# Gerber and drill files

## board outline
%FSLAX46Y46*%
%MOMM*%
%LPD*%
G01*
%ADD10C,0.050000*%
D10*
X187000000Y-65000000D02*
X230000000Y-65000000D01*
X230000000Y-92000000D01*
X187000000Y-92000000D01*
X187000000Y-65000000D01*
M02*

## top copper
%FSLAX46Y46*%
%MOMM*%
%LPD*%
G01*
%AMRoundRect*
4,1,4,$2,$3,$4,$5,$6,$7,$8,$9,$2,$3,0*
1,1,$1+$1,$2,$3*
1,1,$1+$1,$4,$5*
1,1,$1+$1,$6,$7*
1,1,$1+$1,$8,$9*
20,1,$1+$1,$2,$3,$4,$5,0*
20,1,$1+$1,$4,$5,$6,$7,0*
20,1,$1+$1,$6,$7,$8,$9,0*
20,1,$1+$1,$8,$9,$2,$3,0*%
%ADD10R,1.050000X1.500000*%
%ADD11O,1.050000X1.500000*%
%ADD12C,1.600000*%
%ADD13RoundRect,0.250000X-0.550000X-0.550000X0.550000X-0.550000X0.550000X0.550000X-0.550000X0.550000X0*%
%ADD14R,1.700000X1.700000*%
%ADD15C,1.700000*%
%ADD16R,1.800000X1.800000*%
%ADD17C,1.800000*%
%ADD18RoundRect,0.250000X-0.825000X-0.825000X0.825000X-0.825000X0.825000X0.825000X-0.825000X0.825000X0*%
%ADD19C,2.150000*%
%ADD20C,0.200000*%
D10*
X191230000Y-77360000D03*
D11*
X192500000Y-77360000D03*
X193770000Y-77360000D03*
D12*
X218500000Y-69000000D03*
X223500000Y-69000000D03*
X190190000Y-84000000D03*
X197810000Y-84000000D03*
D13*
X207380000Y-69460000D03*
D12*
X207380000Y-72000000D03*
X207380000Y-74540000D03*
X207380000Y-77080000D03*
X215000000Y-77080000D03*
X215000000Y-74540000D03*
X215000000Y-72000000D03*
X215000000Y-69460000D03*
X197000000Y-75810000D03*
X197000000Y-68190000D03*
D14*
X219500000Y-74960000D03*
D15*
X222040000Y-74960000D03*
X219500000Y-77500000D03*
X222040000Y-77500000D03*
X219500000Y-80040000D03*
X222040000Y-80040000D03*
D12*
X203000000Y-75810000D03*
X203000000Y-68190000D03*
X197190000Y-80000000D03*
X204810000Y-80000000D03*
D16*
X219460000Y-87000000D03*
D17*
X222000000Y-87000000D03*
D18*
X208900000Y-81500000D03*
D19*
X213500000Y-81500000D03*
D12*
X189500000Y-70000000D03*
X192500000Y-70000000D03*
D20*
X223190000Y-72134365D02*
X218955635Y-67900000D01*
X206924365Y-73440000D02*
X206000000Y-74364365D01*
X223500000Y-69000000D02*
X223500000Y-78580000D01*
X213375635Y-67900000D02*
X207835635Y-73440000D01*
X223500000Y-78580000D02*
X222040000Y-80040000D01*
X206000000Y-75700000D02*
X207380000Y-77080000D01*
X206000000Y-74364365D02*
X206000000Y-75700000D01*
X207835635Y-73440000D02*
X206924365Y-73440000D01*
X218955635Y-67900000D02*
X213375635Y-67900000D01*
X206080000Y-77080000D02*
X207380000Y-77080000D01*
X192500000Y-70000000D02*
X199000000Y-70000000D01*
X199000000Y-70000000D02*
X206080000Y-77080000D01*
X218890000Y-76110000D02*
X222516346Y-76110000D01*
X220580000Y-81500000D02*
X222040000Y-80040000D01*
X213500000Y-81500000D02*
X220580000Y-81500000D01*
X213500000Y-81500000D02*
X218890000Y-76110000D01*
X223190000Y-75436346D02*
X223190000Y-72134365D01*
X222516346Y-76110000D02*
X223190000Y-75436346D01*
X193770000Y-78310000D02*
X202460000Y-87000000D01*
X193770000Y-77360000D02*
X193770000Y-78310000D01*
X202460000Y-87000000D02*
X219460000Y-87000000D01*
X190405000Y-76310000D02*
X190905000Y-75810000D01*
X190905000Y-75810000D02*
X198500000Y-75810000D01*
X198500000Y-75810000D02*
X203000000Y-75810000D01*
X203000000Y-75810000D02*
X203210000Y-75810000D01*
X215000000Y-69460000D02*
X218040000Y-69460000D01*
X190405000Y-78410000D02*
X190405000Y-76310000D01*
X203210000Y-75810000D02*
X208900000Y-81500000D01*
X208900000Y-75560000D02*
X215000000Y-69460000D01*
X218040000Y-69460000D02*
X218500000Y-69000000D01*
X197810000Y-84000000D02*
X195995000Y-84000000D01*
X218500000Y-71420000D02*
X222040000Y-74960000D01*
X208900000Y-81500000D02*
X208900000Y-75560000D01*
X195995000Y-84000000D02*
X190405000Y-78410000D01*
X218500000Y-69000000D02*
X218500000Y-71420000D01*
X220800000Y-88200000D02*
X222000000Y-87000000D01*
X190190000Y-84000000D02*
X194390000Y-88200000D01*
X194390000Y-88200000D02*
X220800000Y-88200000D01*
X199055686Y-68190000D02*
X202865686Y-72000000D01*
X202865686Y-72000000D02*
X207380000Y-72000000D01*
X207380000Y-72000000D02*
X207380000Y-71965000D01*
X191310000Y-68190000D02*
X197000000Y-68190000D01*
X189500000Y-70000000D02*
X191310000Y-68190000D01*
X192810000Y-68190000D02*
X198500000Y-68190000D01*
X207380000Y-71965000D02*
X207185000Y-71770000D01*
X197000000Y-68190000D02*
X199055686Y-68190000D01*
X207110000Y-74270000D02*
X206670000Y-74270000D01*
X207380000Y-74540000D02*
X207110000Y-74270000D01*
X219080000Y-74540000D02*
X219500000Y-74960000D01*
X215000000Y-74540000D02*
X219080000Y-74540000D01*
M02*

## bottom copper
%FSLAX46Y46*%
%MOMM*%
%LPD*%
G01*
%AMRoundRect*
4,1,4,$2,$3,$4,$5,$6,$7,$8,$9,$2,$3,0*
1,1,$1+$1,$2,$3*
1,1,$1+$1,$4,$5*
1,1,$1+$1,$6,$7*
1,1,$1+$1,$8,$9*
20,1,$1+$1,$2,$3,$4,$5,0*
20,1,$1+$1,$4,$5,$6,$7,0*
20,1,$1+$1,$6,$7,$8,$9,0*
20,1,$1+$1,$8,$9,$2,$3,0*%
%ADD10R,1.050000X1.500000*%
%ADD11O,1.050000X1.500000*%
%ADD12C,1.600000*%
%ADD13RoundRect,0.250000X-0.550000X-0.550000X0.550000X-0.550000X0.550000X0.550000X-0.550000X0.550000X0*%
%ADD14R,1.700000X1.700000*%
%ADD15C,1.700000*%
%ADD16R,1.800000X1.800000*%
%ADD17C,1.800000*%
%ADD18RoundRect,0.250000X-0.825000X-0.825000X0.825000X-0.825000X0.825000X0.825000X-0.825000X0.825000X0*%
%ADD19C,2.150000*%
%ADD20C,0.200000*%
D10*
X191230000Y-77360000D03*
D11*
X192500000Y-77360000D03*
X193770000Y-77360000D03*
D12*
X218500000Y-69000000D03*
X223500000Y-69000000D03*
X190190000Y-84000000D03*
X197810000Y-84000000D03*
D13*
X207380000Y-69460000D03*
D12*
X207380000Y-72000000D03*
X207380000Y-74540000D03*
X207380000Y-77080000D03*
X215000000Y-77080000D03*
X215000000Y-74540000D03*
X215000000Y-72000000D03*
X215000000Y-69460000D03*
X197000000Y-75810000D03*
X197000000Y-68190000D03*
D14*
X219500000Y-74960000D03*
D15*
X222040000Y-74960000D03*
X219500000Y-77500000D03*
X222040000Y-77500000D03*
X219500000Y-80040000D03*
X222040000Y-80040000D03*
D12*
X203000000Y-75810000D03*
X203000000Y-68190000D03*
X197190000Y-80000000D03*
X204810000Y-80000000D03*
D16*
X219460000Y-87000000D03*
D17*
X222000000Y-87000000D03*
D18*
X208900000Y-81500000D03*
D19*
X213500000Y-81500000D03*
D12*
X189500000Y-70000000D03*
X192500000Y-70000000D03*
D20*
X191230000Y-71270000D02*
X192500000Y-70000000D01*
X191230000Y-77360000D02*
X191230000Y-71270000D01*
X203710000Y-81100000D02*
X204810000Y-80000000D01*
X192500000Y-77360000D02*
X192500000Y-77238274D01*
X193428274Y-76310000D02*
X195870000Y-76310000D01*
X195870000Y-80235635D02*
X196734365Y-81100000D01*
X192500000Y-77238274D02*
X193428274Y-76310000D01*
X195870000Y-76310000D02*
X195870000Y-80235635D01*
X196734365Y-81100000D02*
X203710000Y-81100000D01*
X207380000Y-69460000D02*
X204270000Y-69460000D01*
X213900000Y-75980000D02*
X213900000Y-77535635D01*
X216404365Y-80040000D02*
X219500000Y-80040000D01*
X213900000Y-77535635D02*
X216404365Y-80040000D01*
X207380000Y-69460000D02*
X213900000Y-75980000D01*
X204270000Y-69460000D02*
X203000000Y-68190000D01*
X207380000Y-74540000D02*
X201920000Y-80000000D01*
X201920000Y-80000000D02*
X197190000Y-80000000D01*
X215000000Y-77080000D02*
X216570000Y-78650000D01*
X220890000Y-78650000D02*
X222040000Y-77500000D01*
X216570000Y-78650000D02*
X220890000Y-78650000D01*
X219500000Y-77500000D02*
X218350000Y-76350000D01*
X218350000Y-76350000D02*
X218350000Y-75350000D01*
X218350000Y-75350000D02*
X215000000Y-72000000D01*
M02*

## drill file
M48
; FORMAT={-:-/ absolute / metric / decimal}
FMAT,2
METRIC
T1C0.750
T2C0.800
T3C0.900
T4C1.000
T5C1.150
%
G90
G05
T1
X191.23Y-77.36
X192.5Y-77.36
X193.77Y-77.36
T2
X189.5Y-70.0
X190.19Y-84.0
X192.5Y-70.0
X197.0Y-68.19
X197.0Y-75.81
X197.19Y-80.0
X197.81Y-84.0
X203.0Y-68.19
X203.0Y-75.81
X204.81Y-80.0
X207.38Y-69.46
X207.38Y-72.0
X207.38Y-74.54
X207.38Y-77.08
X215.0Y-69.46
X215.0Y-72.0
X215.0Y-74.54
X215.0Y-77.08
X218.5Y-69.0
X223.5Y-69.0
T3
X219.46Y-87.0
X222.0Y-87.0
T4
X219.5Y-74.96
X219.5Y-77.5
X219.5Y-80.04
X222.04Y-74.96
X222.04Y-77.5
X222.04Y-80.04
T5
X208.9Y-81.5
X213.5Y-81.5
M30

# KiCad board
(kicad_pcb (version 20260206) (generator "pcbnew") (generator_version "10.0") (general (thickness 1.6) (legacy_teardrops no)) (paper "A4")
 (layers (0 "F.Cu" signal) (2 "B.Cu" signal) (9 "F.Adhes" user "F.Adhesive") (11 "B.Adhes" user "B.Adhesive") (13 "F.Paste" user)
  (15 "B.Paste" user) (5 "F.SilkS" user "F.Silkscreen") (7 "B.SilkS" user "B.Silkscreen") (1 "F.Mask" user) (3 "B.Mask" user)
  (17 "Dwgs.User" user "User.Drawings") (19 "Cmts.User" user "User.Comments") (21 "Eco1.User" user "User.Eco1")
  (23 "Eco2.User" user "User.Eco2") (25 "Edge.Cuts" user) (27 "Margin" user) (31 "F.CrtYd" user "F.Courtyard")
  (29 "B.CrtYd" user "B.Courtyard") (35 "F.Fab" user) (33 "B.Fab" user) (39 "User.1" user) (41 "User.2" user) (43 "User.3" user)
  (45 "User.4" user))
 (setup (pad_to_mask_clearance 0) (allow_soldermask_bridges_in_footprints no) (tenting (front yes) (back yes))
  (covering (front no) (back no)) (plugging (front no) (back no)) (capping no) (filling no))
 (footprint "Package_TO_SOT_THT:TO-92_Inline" (layer "F.Cu") (at 191.23 77.36)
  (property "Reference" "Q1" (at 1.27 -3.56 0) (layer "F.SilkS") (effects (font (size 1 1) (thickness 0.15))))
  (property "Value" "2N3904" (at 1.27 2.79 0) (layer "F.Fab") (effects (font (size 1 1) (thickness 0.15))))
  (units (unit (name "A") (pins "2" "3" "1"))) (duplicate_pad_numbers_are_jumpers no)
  (pad "1" thru_hole rect (at 0 0) (size 1.05 1.5) (drill 0.75) (layers "*.Cu" "*.Mask") (remove_unused_layers no) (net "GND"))
  (pad "2" thru_hole oval (at 1.27 0) (size 1.05 1.5) (drill 0.75) (layers "*.Cu" "*.Mask") (remove_unused_layers no) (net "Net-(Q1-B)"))
  (pad "3" thru_hole oval (at 2.54 0) (size 1.05 1.5) (drill 0.75) (layers "*.Cu" "*.Mask") (remove_unused_layers no) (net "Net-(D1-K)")))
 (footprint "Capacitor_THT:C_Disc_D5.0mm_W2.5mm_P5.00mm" (layer "F.Cu") (at 218.5 69)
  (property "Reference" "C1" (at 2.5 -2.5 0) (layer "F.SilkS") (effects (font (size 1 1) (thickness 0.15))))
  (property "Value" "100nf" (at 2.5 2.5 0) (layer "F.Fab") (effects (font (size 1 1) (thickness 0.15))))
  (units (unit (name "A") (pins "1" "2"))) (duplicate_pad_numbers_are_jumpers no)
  (pad "1" thru_hole circle (at 0 0) (size 1.6 1.6) (drill 0.8) (layers "*.Cu" "*.Mask") (remove_unused_layers no) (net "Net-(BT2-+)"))
  (pad "2" thru_hole circle (at 5 0) (size 1.6 1.6) (drill 0.8) (layers "*.Cu" "*.Mask") (remove_unused_layers no) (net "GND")))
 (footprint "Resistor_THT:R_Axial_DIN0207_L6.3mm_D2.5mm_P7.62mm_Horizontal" (layer "F.Cu") (at 190.19 84)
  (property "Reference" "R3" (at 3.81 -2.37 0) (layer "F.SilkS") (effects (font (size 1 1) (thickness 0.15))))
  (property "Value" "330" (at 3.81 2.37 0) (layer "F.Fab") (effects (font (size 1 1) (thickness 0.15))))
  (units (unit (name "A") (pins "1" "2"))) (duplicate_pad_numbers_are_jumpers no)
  (pad "1" thru_hole circle (at 0 0) (size 1.6 1.6) (drill 0.8) (layers "*.Cu" "*.Mask") (remove_unused_layers no) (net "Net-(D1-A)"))
  (pad "2" thru_hole circle (at 7.62 0) (size 1.6 1.6) (drill 0.8) (layers "*.Cu" "*.Mask") (remove_unused_layers no) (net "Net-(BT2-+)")))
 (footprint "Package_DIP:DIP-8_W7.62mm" (layer "F.Cu") (at 207.38 69.46)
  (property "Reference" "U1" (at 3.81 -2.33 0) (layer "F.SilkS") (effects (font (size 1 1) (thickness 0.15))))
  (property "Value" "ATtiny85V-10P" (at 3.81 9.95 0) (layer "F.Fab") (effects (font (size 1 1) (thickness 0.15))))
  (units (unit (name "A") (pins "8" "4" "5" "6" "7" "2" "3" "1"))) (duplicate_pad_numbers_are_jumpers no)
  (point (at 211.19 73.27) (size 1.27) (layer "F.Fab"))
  (pad "1" thru_hole roundrect (at 0 0) (size 1.6 1.6) (drill 0.8) (layers "*.Cu" "*.Mask") (remove_unused_layers no)
   (roundrect_rratio 0.15625) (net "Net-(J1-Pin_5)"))
  (pad "2" thru_hole circle (at 0 2.54) (size 1.6 1.6) (drill 0.8) (layers "*.Cu" "*.Mask") (remove_unused_layers no)
   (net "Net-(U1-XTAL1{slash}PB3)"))
  (pad "3" thru_hole circle (at 0 5.08) (size 1.6 1.6) (drill 0.8) (layers "*.Cu" "*.Mask") (remove_unused_layers no)
   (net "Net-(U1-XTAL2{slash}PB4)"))
  (pad "4" thru_hole circle (at 0 7.62) (size 1.6 1.6) (drill 0.8) (layers "*.Cu" "*.Mask") (remove_unused_layers no) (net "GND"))
  (pad "5" thru_hole circle (at 7.62 7.62) (size 1.6 1.6) (drill 0.8) (layers "*.Cu" "*.Mask") (remove_unused_layers no)
   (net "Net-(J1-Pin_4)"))
  (pad "6" thru_hole circle (at 7.62 5.08) (size 1.6 1.6) (drill 0.8) (layers "*.Cu" "*.Mask") (remove_unused_layers no)
   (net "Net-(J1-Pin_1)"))
  (pad "7" thru_hole circle (at 7.62 2.54) (size 1.6 1.6) (drill 0.8) (layers "*.Cu" "*.Mask") (remove_unused_layers no)
   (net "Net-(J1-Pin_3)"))
  (pad "8" thru_hole circle (at 7.62 0) (size 1.6 1.6) (drill 0.8) (layers "*.Cu" "*.Mask") (remove_unused_layers no) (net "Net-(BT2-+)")))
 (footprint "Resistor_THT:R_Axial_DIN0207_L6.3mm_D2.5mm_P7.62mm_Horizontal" (layer "F.Cu") (at 197 75.81 90)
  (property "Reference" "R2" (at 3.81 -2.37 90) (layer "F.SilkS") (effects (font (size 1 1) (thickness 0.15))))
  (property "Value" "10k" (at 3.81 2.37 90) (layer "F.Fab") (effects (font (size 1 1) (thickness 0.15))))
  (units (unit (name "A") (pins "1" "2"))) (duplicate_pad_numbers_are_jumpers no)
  (pad "1" thru_hole circle (at 0 0 90) (size 1.6 1.6) (drill 0.8) (layers "*.Cu" "*.Mask") (remove_unused_layers no) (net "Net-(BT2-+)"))
  (pad "2" thru_hole circle (at 7.62 0 90) (size 1.6 1.6) (drill 0.8) (layers "*.Cu" "*.Mask") (remove_unused_layers no)
   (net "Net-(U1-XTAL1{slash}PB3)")))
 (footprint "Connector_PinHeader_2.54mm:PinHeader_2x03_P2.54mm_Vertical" (layer "F.Cu") (at 219.5 74.96)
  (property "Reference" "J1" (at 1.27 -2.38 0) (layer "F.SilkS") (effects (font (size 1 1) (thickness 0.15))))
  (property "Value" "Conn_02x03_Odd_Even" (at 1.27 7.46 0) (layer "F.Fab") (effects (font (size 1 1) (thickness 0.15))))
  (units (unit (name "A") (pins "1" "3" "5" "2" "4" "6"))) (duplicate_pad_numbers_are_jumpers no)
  (pad "1" thru_hole rect (at 0 0) (size 1.7 1.7) (drill 1) (layers "*.Cu" "*.Mask") (remove_unused_layers no) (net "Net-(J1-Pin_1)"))
  (pad "2" thru_hole circle (at 2.54 0) (size 1.7 1.7) (drill 1) (layers "*.Cu" "*.Mask") (remove_unused_layers no) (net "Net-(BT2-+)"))
  (pad "3" thru_hole circle (at 0 2.54) (size 1.7 1.7) (drill 1) (layers "*.Cu" "*.Mask") (remove_unused_layers no) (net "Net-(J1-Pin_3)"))
  (pad "4" thru_hole circle (at 2.54 2.54) (size 1.7 1.7) (drill 1) (layers "*.Cu" "*.Mask") (remove_unused_layers no)
   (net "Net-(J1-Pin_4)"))
  (pad "5" thru_hole circle (at 0 5.08) (size 1.7 1.7) (drill 1) (layers "*.Cu" "*.Mask") (remove_unused_layers no) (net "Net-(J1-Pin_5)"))
  (pad "6" thru_hole circle (at 2.54 5.08) (size 1.7 1.7) (drill 1) (layers "*.Cu" "*.Mask") (remove_unused_layers no) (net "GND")))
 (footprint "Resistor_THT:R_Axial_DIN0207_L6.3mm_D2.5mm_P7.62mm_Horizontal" (layer "F.Cu") (at 203 75.81 90)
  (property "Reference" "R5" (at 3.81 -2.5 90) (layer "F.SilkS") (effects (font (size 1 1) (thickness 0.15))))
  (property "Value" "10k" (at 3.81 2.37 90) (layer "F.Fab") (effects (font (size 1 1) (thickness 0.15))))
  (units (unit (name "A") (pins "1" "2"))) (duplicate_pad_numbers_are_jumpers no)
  (pad "1" thru_hole circle (at 0 0 90) (size 1.6 1.6) (drill 0.8) (layers "*.Cu" "*.Mask") (remove_unused_layers no) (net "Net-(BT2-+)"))
  (pad "2" thru_hole circle (at 7.62 0 90) (size 1.6 1.6) (drill 0.8) (layers "*.Cu" "*.Mask") (remove_unused_layers no)
   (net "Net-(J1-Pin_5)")))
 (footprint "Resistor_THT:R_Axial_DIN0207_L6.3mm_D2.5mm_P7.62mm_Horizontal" (layer "F.Cu") (at 197.19 80)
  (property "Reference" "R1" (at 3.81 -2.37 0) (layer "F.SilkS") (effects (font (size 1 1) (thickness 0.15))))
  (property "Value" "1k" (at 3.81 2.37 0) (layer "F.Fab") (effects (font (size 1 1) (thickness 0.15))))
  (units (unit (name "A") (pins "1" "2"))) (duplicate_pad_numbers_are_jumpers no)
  (pad "1" thru_hole circle (at 0 0) (size 1.6 1.6) (drill 0.8) (layers "*.Cu" "*.Mask") (remove_unused_layers no)
   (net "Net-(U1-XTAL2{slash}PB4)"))
  (pad "2" thru_hole circle (at 7.62 0) (size 1.6 1.6) (drill 0.8) (layers "*.Cu" "*.Mask") (remove_unused_layers no) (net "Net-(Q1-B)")))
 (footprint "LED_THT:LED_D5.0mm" (layer "F.Cu") (at 219.46 87)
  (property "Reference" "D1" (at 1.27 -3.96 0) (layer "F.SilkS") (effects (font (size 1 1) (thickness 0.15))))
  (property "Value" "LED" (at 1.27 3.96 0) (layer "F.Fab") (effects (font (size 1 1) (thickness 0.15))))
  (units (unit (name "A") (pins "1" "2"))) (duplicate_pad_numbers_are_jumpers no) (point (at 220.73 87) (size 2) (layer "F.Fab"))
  (pad "1" thru_hole rect (at 0 0) (size 1.8 1.8) (drill 0.9) (layers "*.Cu" "*.Mask") (remove_unused_layers no) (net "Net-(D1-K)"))
  (pad "2" thru_hole circle (at 2.54 0) (size 1.8 1.8) (drill 0.9) (layers "*.Cu" "*.Mask") (remove_unused_layers no) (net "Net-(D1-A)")))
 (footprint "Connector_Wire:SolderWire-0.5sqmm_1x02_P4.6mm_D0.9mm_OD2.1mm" (layer "F.Cu") (at 208.9 81.5)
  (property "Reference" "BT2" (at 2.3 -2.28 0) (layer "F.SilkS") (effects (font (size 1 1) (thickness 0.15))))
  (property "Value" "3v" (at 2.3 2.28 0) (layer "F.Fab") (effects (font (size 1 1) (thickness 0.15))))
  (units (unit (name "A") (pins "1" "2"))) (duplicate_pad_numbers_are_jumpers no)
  (pad "1" thru_hole roundrect (at 0 0) (size 2.15 2.15) (drill 1.15) (layers "*.Cu" "*.Mask") (remove_unused_layers no)
   (roundrect_rratio 0.116279) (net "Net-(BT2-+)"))
  (pad "2" thru_hole circle (at 4.6 0) (size 2.15 2.15) (drill 1.15) (layers "*.Cu" "*.Mask") (remove_unused_layers no) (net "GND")))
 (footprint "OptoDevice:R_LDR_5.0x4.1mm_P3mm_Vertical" (layer "F.Cu") (at 189.5 70)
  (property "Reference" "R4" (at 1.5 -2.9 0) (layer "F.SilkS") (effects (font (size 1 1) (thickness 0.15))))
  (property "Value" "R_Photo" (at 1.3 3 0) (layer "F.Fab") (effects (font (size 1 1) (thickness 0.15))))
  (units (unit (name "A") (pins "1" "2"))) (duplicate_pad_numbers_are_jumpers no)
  (pad "1" thru_hole circle (at 0 0) (size 1.6 1.6) (drill 0.8) (layers "*.Cu" "*.Mask") (remove_unused_layers no)
   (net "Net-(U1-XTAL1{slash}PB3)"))
  (pad "2" thru_hole circle (at 3 0) (size 1.6 1.6) (drill 0.8) (layers "*.Cu" "*.Mask") (remove_unused_layers no) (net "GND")))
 (gr_rect (start 187 65) (end 230 92) (stroke (width 0.05) (type default)) (fill no) (layer "Edge.Cuts"))
 (segment (start 223.19 72.134365) (end 218.955635 67.9) (width 0.2) (layer "F.Cu") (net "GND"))
 (segment (start 206.924365 73.44) (end 206 74.364365) (width 0.2) (layer "F.Cu") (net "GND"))
 (segment (start 223.5 69) (end 223.5 78.58) (width 0.2) (layer "F.Cu") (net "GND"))
 (segment (start 213.375635 67.9) (end 207.835635 73.44) (width 0.2) (layer "F.Cu") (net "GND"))
 (segment (start 223.5 78.58) (end 222.04 80.04) (width 0.2) (layer "F.Cu") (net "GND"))
 (segment (start 206 75.7) (end 207.38 77.08) (width 0.2) (layer "F.Cu") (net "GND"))
 (segment (start 206 74.364365) (end 206 75.7) (width 0.2) (layer "F.Cu") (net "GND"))
 (segment (start 207.835635 73.44) (end 206.924365 73.44) (width 0.2) (layer "F.Cu") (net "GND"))
 (segment (start 218.955635 67.9) (end 213.375635 67.9) (width 0.2) (layer "F.Cu") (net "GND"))
 (segment (start 206.08 77.08) (end 207.38 77.08) (width 0.2) (layer "F.Cu") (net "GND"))
 (segment (start 192.5 70) (end 199 70) (width 0.2) (layer "F.Cu") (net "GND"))
 (segment (start 199 70) (end 206.08 77.08) (width 0.2) (layer "F.Cu") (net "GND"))
 (segment (start 218.89 76.11) (end 222.516346 76.11) (width 0.2) (layer "F.Cu") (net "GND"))
 (segment (start 220.58 81.5) (end 222.04 80.04) (width 0.2) (layer "F.Cu") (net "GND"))
 (segment (start 213.5 81.5) (end 220.58 81.5) (width 0.2) (layer "F.Cu") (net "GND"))
 (segment (start 213.5 81.5) (end 218.89 76.11) (width 0.2) (layer "F.Cu") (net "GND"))
 (segment (start 223.19 75.436346) (end 223.19 72.134365) (width 0.2) (layer "F.Cu") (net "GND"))
 (segment (start 222.516346 76.11) (end 223.19 75.436346) (width 0.2) (layer "F.Cu") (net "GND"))
 (segment (start 191.23 71.27) (end 192.5 70) (width 0.2) (layer "B.Cu") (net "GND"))
 (segment (start 191.23 77.36) (end 191.23 71.27) (width 0.2) (layer "B.Cu") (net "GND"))
 (segment (start 203.71 81.1) (end 204.81 80) (width 0.2) (layer "B.Cu") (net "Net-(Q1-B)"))
 (segment (start 192.5 77.36) (end 192.5 77.238274) (width 0.2) (layer "B.Cu") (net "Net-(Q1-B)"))
 (segment (start 193.428274 76.31) (end 195.87 76.31) (width 0.2) (layer "B.Cu") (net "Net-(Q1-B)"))
 (segment (start 195.87 80.235635) (end 196.734365 81.1) (width 0.2) (layer "B.Cu") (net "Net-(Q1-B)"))
 (segment (start 192.5 77.238274) (end 193.428274 76.31) (width 0.2) (layer "B.Cu") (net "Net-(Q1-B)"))
 (segment (start 195.87 76.31) (end 195.87 80.235635) (width 0.2) (layer "B.Cu") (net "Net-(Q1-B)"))
 (segment (start 196.734365 81.1) (end 203.71 81.1) (width 0.2) (layer "B.Cu") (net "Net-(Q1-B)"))
 (segment (start 193.77 78.31) (end 202.46 87) (width 0.2) (layer "F.Cu") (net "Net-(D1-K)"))
 (segment (start 193.77 77.36) (end 193.77 78.31) (width 0.2) (layer "F.Cu") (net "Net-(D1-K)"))
 (segment (start 202.46 87) (end 219.46 87) (width 0.2) (layer "F.Cu") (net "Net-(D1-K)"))
 (segment (start 190.405 76.31) (end 190.905 75.81) (width 0.2) (layer "F.Cu") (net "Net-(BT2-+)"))
 (segment (start 190.905 75.81) (end 198.5 75.81) (width 0.2) (layer "F.Cu") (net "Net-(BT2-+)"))
 (segment (start 198.5 75.81) (end 203 75.81) (width 0.2) (layer "F.Cu") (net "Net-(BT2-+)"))
 (segment (start 203 75.81) (end 203.21 75.81) (width 0.2) (layer "F.Cu") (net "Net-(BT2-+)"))
 (segment (start 215 69.46) (end 218.04 69.46) (width 0.2) (layer "F.Cu") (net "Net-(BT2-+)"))
 (segment (start 190.405 78.41) (end 190.405 76.31) (width 0.2) (layer "F.Cu") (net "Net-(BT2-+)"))
 (segment (start 203.21 75.81) (end 208.9 81.5) (width 0.2) (layer "F.Cu") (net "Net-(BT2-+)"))
 (segment (start 208.9 75.56) (end 215 69.46) (width 0.2) (layer "F.Cu") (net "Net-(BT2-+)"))
 (segment (start 218.04 69.46) (end 218.5 69) (width 0.2) (layer "F.Cu") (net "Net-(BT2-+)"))
 (segment (start 197.81 84) (end 195.995 84) (width 0.2) (layer "F.Cu") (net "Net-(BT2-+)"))
 (segment (start 218.5 71.42) (end 222.04 74.96) (width 0.2) (layer "F.Cu") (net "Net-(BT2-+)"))
 (segment (start 208.9 81.5) (end 208.9 75.56) (width 0.2) (layer "F.Cu") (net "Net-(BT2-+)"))
 (segment (start 195.995 84) (end 190.405 78.41) (width 0.2) (layer "F.Cu") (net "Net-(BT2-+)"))
 (segment (start 218.5 69) (end 218.5 71.42) (width 0.2) (layer "F.Cu") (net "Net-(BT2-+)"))
 (segment (start 220.8 88.2) (end 222 87) (width 0.2) (layer "F.Cu") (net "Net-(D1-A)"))
 (segment (start 190.19 84) (end 194.39 88.2) (width 0.2) (layer "F.Cu") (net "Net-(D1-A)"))
 (segment (start 194.39 88.2) (end 220.8 88.2) (width 0.2) (layer "F.Cu") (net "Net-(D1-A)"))
 (segment (start 207.38 69.46) (end 204.27 69.46) (width 0.2) (layer "B.Cu") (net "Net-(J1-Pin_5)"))
 (segment (start 213.9 75.98) (end 213.9 77.535635) (width 0.2) (layer "B.Cu") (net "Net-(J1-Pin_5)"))
 (segment (start 216.404365 80.04) (end 219.5 80.04) (width 0.2) (layer "B.Cu") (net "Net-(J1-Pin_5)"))
 (segment (start 213.9 77.535635) (end 216.404365 80.04) (width 0.2) (layer "B.Cu") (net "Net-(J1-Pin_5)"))
 (segment (start 207.38 69.46) (end 213.9 75.98) (width 0.2) (layer "B.Cu") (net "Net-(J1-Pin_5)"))
 (segment (start 204.27 69.46) (end 203 68.19) (width 0.2) (layer "B.Cu") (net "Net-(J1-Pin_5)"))
 (segment (start 199.055686 68.19) (end 202.865686 72) (width 0.2) (layer "F.Cu") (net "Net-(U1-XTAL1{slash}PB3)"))
 (segment (start 202.865686 72) (end 207.38 72) (width 0.2) (layer "F.Cu") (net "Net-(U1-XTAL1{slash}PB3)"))
 (segment (start 207.38 72) (end 207.38 71.965) (width 0.2) (layer "F.Cu") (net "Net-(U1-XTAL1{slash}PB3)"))
 (segment (start 191.31 68.19) (end 197 68.19) (width 0.2) (layer "F.Cu") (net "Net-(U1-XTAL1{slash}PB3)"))
 (segment (start 189.5 70) (end 191.31 68.19) (width 0.2) (layer "F.Cu") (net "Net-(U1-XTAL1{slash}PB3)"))
 (segment (start 192.81 68.19) (end 198.5 68.19) (width 0.2) (layer "F.Cu") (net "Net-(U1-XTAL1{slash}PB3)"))
 (segment (start 207.38 71.965) (end 207.185 71.77) (width 0.2) (layer "F.Cu") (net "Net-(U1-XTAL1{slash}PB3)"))
 (segment (start 197 68.19) (end 199.055686 68.19) (width 0.2) (layer "F.Cu") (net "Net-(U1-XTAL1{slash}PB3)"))
 (segment (start 207.11 74.27) (end 206.67 74.27) (width 0.2) (layer "F.Cu") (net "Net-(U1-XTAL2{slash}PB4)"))
 (segment (start 207.38 74.54) (end 207.11 74.27) (width 0.2) (layer "F.Cu") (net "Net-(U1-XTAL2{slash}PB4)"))
 (segment (start 207.38 74.54) (end 201.92 80) (width 0.2) (layer "B.Cu") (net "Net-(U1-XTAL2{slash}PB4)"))
 (segment (start 201.92 80) (end 197.19 80) (width 0.2) (layer "B.Cu") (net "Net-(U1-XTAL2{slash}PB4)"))
 (segment (start 215 77.08) (end 216.57 78.65) (width 0.2) (layer "B.Cu") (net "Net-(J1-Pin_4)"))
 (segment (start 220.89 78.65) (end 222.04 77.5) (width 0.2) (layer "B.Cu") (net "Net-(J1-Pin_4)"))
 (segment (start 216.57 78.65) (end 220.89 78.65) (width 0.2) (layer "B.Cu") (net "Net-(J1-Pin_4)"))
 (segment (start 219.08 74.54) (end 219.5 74.96) (width 0.2) (layer "F.Cu") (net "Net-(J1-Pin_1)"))
 (segment (start 215 74.54) (end 219.08 74.54) (width 0.2) (layer "F.Cu") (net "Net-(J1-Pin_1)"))
 (segment (start 219.5 77.5) (end 218.35 76.35) (width 0.2) (layer "B.Cu") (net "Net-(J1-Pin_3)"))
 (segment (start 218.35 76.35) (end 218.35 75.35) (width 0.2) (layer "B.Cu") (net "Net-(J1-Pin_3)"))
 (segment (start 218.35 75.35) (end 215 72) (width 0.2) (layer "B.Cu") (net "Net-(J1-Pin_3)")))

